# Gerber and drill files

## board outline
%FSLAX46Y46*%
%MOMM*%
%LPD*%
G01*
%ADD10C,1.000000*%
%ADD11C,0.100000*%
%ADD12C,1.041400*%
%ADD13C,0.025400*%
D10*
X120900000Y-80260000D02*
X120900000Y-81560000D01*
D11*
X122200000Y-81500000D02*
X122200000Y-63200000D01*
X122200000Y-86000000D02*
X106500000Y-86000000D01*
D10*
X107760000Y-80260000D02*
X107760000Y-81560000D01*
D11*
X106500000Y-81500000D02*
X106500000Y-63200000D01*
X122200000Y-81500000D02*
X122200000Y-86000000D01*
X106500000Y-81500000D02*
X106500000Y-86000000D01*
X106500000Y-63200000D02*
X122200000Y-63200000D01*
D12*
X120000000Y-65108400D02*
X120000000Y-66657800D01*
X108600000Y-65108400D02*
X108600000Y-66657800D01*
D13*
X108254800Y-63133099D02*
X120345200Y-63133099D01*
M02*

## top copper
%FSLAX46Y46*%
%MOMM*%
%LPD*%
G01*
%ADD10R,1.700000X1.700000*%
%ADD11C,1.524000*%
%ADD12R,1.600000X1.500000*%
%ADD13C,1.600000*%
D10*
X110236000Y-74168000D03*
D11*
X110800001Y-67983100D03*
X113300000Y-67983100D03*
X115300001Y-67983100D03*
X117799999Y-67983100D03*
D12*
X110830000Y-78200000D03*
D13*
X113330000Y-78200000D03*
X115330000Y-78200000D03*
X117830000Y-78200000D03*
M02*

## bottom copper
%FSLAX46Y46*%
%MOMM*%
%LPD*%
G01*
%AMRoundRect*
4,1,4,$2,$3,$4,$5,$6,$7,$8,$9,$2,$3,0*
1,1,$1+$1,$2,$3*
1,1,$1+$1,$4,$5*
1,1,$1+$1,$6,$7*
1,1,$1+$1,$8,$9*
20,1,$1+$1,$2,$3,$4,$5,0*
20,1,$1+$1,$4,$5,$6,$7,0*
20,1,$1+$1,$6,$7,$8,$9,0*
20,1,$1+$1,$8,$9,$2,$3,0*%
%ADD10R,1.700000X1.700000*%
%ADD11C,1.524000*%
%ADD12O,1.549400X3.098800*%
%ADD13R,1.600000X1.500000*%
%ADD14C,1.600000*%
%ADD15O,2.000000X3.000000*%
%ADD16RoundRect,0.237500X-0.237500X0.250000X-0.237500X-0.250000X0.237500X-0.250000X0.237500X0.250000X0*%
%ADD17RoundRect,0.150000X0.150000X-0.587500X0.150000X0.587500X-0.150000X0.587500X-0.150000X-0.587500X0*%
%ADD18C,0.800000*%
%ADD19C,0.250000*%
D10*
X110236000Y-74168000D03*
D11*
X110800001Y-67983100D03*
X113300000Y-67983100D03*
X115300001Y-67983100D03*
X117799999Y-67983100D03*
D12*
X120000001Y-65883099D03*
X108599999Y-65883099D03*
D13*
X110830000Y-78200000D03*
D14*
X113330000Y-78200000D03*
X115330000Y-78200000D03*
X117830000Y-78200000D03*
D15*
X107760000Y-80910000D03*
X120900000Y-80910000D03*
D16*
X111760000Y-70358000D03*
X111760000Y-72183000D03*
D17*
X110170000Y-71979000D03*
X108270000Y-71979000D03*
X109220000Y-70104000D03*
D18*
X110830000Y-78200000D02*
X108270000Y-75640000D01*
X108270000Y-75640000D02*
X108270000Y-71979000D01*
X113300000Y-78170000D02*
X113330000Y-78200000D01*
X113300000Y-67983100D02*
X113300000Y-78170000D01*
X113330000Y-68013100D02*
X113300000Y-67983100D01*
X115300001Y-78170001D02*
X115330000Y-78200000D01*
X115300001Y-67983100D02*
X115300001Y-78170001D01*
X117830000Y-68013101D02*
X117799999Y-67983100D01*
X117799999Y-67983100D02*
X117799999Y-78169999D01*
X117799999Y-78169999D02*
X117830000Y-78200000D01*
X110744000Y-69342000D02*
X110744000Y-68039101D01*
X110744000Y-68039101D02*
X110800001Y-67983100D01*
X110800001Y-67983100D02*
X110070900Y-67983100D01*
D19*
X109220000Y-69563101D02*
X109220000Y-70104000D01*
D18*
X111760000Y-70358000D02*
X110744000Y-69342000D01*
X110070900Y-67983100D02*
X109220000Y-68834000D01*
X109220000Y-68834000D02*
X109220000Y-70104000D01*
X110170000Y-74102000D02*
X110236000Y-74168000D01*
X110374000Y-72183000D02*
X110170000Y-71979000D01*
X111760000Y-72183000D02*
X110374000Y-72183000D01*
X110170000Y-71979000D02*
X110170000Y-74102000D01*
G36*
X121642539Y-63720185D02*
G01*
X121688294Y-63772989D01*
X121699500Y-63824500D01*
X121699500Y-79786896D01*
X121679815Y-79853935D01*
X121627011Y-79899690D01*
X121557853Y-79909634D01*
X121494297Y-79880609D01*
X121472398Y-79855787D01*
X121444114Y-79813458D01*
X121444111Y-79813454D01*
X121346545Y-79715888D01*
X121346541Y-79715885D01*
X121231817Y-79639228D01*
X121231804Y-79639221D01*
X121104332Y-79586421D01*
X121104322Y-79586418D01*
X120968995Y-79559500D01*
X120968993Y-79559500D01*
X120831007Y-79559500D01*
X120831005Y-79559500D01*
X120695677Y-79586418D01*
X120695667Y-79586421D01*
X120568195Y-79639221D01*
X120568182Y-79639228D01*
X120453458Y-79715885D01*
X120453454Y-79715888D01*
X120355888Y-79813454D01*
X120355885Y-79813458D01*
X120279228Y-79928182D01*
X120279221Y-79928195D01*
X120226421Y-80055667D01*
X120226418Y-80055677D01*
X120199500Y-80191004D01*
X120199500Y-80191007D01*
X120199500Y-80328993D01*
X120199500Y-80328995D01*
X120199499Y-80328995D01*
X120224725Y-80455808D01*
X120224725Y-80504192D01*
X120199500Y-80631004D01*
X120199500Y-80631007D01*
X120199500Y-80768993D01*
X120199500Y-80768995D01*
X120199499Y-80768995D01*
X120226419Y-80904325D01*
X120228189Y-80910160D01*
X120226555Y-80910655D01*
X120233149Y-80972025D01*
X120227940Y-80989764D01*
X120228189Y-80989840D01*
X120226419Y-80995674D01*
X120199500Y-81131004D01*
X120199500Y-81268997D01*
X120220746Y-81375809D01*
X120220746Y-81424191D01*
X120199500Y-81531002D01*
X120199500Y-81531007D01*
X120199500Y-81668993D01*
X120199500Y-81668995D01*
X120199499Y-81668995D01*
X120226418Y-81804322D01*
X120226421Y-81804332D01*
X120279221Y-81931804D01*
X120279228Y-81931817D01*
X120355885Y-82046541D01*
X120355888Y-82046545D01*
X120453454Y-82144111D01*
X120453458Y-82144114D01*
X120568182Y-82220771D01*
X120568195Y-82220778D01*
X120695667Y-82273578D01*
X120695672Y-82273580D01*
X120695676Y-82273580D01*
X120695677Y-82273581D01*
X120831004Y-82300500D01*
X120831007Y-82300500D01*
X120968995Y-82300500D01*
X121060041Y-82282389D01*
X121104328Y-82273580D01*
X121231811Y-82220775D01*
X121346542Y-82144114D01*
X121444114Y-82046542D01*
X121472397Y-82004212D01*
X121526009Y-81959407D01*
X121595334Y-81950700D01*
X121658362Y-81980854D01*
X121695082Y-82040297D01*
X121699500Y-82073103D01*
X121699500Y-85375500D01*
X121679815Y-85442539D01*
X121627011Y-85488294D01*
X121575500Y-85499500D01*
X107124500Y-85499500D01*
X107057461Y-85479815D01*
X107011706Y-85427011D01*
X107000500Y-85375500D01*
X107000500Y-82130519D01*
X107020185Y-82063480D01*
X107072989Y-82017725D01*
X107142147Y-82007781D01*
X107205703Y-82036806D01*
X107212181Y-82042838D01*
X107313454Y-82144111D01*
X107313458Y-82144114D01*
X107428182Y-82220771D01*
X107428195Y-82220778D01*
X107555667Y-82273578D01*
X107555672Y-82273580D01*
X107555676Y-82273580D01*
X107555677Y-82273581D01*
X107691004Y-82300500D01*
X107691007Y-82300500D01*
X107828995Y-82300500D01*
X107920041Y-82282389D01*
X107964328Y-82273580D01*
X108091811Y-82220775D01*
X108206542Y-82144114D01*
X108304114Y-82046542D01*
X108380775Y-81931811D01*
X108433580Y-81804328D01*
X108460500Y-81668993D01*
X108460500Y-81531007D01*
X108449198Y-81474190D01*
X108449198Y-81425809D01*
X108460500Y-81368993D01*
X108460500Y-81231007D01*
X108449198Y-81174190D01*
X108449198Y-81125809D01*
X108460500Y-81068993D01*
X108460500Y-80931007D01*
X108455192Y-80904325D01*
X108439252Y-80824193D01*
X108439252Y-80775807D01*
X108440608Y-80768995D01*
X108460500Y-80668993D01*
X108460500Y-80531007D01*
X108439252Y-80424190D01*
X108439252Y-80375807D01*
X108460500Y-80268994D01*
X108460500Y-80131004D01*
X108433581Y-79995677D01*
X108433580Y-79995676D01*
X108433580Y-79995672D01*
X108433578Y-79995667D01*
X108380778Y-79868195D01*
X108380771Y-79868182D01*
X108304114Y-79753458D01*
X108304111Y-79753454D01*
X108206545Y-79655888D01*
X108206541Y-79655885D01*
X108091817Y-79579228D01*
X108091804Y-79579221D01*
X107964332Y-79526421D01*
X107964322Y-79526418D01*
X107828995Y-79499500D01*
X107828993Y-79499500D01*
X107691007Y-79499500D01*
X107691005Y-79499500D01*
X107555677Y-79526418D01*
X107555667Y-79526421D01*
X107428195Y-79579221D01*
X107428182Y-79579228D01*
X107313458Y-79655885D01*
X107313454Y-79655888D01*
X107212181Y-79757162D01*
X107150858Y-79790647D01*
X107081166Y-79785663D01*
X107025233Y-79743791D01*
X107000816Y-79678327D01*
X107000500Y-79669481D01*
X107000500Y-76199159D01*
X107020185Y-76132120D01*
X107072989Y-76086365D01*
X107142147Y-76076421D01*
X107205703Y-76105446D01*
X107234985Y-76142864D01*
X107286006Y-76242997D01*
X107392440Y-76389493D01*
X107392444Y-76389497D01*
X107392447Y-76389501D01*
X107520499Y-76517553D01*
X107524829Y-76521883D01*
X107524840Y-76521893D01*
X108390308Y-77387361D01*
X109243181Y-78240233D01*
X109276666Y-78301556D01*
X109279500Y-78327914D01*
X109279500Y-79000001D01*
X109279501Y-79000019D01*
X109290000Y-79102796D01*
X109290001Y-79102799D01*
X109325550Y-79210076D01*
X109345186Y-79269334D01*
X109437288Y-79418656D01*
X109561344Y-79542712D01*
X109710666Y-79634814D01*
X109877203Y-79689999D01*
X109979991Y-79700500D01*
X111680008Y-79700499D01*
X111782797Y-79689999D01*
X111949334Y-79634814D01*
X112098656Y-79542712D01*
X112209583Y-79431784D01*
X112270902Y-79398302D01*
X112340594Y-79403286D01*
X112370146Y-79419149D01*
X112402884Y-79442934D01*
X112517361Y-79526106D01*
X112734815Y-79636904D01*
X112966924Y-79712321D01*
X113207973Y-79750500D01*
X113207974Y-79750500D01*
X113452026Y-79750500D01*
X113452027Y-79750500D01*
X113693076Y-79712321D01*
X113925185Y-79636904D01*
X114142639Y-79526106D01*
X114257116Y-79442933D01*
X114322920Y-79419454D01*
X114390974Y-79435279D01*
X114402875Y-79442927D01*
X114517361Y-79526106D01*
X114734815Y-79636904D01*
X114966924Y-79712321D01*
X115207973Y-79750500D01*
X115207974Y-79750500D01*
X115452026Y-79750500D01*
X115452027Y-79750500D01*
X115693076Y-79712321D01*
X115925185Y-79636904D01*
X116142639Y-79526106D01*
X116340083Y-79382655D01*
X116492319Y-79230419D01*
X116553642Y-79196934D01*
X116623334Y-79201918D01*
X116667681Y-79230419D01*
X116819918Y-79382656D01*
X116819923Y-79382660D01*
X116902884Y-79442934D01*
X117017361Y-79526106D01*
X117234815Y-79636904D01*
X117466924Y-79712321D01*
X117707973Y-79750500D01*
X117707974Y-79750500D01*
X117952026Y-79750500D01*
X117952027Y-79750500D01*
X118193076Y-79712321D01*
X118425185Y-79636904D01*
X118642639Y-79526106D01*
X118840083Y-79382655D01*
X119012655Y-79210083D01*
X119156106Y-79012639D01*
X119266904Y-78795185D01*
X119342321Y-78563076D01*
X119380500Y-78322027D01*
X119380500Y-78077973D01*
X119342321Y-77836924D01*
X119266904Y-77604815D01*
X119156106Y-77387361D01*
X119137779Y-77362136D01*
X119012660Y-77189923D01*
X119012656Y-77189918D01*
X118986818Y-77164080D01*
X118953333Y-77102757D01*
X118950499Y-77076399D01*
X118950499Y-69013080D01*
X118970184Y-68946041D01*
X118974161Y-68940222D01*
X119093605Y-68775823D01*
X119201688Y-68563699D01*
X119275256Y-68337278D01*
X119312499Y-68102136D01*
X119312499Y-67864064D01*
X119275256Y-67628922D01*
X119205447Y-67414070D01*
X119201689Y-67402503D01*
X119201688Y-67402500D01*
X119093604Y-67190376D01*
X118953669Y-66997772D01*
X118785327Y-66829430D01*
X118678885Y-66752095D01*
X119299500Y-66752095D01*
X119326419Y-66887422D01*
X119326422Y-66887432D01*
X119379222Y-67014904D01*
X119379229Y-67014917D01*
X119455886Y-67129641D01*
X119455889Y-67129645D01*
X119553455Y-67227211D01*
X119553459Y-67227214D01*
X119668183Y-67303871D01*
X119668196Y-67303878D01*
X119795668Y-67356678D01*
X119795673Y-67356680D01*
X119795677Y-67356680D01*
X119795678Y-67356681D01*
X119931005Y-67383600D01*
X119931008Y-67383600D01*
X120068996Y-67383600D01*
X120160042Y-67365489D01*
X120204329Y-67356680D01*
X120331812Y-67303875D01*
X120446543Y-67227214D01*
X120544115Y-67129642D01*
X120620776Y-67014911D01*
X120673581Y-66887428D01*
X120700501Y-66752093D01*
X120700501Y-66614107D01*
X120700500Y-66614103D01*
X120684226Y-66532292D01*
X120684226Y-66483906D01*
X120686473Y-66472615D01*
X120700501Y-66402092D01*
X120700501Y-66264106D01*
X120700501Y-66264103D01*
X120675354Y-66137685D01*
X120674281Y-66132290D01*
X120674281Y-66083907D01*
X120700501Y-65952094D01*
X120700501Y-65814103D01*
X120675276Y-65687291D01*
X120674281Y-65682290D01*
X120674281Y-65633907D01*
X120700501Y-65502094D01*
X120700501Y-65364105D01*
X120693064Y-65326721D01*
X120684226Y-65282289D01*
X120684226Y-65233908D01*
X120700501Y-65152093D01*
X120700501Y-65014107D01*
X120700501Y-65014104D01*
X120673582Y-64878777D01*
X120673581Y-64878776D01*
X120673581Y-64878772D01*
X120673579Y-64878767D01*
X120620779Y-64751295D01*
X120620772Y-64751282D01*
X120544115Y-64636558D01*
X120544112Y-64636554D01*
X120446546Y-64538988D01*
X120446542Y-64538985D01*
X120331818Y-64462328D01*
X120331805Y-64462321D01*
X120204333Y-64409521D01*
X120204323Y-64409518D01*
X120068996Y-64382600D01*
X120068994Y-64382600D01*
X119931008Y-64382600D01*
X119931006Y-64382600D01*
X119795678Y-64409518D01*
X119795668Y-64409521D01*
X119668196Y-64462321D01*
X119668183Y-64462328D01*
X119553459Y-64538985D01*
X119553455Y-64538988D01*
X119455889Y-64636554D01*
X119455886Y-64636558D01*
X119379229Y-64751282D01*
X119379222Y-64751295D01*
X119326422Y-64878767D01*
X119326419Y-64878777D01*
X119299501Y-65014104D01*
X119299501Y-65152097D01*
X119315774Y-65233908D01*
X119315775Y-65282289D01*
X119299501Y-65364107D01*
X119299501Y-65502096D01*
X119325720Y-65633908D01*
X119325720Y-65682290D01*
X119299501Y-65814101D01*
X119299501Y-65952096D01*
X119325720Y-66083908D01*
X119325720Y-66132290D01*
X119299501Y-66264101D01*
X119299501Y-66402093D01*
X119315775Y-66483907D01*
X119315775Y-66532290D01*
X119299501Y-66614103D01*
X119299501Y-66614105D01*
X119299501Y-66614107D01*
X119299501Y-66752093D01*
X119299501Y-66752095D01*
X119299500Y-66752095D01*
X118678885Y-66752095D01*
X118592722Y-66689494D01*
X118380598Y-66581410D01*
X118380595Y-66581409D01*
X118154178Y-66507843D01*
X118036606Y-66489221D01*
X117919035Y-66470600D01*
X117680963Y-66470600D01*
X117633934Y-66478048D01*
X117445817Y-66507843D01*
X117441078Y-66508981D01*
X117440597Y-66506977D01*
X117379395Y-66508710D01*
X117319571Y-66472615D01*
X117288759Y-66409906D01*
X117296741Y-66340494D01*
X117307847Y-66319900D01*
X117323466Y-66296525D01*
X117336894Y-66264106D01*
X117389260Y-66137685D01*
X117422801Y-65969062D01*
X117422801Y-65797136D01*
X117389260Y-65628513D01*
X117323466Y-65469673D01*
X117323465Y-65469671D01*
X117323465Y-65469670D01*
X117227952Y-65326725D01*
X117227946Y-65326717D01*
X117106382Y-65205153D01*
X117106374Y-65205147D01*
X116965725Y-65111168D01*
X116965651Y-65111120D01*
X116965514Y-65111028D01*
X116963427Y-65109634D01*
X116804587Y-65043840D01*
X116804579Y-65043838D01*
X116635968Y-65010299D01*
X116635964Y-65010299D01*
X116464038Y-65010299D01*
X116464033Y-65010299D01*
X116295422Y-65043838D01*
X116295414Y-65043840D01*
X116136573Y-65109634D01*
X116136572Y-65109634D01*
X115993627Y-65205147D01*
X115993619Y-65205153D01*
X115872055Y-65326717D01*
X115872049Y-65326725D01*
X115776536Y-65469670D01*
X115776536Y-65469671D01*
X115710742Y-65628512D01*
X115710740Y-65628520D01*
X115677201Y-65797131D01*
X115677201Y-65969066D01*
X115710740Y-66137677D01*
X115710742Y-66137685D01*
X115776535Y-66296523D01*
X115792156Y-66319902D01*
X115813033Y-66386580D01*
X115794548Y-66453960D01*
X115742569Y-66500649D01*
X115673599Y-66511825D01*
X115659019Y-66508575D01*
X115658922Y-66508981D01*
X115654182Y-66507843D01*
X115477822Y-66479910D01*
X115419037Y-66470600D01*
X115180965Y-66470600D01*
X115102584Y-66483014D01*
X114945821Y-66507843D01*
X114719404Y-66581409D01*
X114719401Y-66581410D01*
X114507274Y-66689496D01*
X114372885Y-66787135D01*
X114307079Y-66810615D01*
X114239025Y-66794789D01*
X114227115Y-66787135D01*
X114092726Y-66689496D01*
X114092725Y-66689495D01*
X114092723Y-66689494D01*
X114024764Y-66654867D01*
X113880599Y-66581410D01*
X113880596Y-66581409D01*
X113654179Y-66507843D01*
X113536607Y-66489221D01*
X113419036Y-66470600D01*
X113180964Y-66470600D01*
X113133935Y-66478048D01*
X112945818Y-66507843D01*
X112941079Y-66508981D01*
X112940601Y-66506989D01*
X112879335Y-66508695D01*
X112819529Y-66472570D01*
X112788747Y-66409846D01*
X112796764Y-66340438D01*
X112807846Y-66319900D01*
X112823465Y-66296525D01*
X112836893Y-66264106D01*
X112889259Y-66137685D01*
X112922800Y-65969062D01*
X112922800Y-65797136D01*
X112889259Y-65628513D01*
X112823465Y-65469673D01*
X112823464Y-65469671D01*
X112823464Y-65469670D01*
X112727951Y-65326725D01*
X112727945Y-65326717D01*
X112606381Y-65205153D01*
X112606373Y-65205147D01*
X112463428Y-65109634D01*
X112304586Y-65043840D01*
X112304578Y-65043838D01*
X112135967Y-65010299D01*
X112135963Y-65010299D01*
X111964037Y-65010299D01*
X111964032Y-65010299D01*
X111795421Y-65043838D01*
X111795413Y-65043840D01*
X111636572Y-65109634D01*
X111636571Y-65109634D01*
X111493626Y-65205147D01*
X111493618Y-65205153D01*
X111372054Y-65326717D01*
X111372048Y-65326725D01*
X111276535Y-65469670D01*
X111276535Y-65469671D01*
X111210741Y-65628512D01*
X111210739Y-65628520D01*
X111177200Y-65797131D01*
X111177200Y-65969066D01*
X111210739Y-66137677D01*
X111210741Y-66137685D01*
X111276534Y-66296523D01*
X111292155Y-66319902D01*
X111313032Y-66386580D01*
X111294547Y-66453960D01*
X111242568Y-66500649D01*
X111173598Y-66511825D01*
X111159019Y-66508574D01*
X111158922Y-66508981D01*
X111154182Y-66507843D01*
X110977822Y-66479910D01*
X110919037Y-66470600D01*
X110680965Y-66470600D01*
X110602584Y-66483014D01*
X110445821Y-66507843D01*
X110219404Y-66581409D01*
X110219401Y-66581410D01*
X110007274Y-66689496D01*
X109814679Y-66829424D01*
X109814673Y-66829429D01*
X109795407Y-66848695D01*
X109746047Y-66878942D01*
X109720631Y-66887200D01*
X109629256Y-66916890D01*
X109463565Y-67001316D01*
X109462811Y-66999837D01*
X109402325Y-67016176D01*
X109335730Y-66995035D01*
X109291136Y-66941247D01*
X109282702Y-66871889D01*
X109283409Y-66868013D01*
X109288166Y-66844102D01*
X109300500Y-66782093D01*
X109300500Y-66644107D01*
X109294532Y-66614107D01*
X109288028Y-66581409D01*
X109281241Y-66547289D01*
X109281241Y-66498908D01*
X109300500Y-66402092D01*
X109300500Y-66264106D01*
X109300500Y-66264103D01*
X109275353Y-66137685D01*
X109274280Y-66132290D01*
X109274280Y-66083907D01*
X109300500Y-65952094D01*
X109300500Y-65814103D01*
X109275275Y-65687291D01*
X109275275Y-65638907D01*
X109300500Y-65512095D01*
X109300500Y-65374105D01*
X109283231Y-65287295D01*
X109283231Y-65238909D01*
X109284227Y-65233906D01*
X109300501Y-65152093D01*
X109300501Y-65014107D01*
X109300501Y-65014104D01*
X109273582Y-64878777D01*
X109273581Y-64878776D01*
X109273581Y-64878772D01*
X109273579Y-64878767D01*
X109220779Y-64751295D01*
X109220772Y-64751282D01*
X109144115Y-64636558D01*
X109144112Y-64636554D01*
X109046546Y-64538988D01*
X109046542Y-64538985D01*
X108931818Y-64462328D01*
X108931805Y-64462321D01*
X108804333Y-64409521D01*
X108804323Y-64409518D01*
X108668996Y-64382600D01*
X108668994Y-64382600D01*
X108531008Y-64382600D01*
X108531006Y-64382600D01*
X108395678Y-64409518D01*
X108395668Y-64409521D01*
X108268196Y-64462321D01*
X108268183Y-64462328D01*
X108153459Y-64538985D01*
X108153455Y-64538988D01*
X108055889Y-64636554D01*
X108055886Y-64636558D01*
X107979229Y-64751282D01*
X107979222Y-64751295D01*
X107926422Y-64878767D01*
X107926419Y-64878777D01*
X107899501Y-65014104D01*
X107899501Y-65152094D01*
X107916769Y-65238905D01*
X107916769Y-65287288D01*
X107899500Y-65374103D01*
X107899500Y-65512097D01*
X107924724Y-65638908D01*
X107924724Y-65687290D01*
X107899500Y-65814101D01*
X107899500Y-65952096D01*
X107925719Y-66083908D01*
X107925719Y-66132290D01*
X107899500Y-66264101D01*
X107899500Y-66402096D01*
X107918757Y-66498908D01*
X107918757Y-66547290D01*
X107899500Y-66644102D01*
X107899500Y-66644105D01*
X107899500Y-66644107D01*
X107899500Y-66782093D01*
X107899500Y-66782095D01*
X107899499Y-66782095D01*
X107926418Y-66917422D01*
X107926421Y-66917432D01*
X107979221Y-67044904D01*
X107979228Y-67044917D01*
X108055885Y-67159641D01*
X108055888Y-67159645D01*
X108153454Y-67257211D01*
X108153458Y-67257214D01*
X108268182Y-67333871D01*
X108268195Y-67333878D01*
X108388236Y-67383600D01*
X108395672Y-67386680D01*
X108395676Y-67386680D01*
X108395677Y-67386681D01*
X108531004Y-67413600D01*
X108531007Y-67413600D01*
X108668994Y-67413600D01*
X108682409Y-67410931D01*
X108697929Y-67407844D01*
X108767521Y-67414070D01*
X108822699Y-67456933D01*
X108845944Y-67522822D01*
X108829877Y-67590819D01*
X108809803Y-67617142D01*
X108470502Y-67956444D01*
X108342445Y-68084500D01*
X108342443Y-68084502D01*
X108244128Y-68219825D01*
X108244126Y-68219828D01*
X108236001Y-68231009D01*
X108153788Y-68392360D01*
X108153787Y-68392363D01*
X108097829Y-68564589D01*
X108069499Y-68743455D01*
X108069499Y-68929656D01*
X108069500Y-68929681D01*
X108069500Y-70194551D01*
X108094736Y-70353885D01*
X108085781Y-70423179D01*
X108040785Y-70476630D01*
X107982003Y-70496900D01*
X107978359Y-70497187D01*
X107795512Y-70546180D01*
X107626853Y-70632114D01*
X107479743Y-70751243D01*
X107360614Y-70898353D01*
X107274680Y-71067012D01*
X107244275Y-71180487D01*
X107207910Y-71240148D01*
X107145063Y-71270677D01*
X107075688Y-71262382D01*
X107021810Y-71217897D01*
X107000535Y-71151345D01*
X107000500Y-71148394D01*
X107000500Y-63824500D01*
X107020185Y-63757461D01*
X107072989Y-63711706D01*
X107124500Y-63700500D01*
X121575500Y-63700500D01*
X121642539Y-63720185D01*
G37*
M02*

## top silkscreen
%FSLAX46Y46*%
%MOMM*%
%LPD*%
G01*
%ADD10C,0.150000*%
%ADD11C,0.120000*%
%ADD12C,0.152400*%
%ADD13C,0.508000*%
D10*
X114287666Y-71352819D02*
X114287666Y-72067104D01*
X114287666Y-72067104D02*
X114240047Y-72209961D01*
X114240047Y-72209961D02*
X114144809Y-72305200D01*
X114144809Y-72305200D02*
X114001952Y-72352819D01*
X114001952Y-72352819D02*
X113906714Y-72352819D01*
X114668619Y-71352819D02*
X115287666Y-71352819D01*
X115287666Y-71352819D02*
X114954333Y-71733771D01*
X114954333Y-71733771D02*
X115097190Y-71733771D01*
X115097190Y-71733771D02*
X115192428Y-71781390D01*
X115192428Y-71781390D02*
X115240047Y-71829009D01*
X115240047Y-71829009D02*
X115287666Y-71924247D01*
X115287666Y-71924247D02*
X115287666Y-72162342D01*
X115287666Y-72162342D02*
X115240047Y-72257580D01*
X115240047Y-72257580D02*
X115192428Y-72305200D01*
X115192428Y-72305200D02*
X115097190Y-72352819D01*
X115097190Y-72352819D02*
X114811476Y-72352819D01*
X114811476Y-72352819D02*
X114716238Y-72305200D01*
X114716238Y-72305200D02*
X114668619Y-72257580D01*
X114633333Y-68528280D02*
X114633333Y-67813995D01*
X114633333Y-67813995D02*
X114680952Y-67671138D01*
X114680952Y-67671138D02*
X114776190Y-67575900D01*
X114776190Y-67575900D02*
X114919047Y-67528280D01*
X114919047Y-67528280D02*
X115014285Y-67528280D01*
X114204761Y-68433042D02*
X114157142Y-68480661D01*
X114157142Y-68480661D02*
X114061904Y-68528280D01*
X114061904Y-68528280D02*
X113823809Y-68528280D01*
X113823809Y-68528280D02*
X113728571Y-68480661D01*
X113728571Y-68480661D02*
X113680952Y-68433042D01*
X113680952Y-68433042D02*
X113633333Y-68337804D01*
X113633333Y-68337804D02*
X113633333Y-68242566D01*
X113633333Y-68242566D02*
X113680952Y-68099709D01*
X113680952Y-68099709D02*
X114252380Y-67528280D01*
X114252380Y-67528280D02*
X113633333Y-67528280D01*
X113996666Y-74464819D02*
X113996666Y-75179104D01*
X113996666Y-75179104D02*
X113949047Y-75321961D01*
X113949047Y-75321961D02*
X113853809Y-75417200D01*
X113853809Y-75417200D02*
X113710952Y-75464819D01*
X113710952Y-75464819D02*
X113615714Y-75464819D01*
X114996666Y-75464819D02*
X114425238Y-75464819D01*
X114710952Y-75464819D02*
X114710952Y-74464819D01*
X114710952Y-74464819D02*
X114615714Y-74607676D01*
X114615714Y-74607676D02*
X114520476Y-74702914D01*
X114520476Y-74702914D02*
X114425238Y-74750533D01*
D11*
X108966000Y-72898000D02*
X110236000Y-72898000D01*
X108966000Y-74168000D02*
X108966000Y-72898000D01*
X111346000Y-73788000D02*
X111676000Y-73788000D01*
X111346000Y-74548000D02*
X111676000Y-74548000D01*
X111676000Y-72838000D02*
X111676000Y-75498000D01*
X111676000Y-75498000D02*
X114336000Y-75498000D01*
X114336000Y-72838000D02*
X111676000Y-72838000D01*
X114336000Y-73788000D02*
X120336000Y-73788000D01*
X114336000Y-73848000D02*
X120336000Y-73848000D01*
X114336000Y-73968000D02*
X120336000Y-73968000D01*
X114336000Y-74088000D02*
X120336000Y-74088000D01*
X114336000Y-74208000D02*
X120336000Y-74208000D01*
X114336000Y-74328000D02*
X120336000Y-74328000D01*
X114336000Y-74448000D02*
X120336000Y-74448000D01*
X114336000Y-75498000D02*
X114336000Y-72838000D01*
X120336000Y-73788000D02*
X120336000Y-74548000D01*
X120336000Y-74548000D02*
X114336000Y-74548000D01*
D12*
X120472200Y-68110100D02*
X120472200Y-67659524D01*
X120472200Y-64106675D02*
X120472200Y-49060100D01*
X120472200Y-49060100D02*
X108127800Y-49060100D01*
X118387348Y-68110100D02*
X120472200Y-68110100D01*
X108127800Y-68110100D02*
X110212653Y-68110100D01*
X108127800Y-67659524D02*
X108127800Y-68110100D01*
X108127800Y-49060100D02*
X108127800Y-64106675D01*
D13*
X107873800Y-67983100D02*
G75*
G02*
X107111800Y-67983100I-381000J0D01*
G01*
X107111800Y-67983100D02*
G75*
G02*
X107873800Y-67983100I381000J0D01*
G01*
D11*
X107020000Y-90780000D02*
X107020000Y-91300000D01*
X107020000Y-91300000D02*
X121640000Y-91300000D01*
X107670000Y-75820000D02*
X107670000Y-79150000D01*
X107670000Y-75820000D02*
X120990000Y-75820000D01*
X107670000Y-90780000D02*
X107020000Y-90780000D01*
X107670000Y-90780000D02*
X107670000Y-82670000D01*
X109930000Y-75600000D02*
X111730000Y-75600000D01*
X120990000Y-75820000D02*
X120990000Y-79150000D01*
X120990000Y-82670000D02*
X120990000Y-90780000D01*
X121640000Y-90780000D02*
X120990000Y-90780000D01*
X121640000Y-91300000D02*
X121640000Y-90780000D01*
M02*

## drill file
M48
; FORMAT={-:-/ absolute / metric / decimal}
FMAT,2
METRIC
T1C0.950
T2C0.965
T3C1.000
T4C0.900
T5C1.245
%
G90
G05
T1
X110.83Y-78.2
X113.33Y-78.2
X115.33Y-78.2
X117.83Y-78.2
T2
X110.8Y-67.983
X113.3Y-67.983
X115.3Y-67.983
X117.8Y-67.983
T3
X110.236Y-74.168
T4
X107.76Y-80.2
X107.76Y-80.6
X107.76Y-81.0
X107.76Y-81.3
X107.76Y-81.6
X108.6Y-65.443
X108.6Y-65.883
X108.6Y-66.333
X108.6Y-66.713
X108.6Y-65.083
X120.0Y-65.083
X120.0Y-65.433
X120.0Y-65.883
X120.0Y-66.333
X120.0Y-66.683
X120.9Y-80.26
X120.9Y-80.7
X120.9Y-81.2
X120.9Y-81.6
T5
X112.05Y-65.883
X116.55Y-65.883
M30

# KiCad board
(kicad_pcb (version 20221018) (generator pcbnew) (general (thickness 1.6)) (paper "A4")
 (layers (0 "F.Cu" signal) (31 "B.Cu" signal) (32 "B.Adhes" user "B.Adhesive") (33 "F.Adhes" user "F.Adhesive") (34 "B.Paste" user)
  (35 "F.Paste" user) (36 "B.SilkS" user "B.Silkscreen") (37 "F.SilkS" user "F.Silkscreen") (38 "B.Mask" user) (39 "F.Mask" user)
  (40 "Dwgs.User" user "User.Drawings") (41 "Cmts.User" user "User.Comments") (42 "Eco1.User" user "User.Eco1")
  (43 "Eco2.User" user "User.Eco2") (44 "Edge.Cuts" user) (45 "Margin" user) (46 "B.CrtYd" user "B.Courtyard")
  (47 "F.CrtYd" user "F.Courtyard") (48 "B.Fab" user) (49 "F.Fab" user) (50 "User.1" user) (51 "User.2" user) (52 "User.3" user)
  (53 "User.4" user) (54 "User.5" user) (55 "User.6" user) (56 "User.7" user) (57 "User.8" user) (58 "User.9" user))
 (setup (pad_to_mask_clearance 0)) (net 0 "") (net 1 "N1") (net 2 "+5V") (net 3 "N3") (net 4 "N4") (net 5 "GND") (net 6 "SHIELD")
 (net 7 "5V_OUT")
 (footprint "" (layer "F.Cu") (at 120.9 78.74)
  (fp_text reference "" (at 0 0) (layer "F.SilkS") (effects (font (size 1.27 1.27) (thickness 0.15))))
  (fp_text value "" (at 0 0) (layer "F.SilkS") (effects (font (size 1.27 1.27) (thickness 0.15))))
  (pad "" np_thru_hole circle (at 0 1.96 180) (size 0.9 0.9) (drill 0.9) (layers "F&B.Cu" "*.Mask")))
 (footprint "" (layer "F.Cu") (at 120.9 79.24)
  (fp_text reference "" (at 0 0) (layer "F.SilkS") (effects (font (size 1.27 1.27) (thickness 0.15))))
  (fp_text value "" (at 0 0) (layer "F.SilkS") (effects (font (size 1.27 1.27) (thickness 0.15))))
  (pad "" np_thru_hole circle (at 0 1.96 180) (size 0.9 0.9) (drill 0.9) (layers "F&B.Cu" "*.Mask")))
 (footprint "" (layer "F.Cu") (at 104.2 78.24)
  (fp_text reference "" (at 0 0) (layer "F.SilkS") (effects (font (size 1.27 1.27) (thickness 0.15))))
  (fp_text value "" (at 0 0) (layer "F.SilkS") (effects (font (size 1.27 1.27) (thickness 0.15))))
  (pad "" np_thru_hole circle (at 3.56 1.96 180) (size 0.9 0.9) (drill 0.9) (layers "F&B.Cu" "*.Mask")))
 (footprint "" (layer "F.Cu") (at 120.9 79.64)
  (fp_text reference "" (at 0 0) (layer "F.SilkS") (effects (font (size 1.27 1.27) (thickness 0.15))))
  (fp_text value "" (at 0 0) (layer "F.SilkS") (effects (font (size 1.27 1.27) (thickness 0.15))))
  (pad "" np_thru_hole circle (at 0 1.96 180) (size 0.9 0.9) (drill 0.9) (layers "F&B.Cu" "*.Mask")))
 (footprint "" (layer "F.Cu") (at 104.2 78.64)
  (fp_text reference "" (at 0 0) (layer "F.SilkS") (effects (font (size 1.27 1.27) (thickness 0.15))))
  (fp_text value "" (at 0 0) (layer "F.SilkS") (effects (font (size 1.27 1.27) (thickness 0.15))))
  (pad "" np_thru_hole circle (at 3.56 1.96 180) (size 0.9 0.9) (drill 0.9) (layers "F&B.Cu" "*.Mask")))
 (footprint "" (layer "F.Cu") (at 120.9 78.3)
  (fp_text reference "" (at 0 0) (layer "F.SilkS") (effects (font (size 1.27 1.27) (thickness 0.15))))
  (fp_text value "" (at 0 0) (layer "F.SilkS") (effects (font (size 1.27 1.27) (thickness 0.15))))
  (pad "" np_thru_hole circle (at 0 1.96 180) (size 0.9 0.9) (drill 0.9) (layers "F&B.Cu" "*.Mask")))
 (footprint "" (layer "F.Cu") (at 104.2 79.34)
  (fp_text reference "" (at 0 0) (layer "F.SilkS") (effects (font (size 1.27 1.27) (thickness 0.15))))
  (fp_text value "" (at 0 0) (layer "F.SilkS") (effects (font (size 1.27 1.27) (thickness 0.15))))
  (pad "" np_thru_hole circle (at 3.56 1.96 180) (size 0.9 0.9) (drill 0.9) (layers "F&B.Cu" "*.Mask")))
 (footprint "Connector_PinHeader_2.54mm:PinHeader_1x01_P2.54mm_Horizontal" (layer "F.Cu") (at 110.236 74.168)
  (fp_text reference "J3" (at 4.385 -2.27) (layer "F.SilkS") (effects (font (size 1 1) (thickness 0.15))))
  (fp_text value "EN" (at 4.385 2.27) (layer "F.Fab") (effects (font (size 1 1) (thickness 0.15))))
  (fp_line (start -1.27 -1.27) (end 0 -1.27) (stroke (width 0.12) (type solid)) (layer "F.SilkS"))
  (fp_line (start -1.27 0) (end -1.27 -1.27) (stroke (width 0.12) (type solid)) (layer "F.SilkS"))
  (fp_line (start 1.11 -0.38) (end 1.44 -0.38) (stroke (width 0.12) (type solid)) (layer "F.SilkS"))
  (fp_line (start 1.11 0.38) (end 1.44 0.38) (stroke (width 0.12) (type solid)) (layer "F.SilkS"))
  (fp_line (start 1.44 -1.33) (end 1.44 1.33) (stroke (width 0.12) (type solid)) (layer "F.SilkS"))
  (fp_line (start 1.44 1.33) (end 4.1 1.33) (stroke (width 0.12) (type solid)) (layer "F.SilkS"))
  (fp_line (start 4.1 -1.33) (end 1.44 -1.33) (stroke (width 0.12) (type solid)) (layer "F.SilkS"))
  (fp_line (start 4.1 -0.38) (end 10.1 -0.38) (stroke (width 0.12) (type solid)) (layer "F.SilkS"))
  (fp_line (start 4.1 -0.32) (end 10.1 -0.32) (stroke (width 0.12) (type solid)) (layer "F.SilkS"))
  (fp_line (start 4.1 -0.2) (end 10.1 -0.2) (stroke (width 0.12) (type solid)) (layer "F.SilkS"))
  (fp_line (start 4.1 -0.08) (end 10.1 -0.08) (stroke (width 0.12) (type solid)) (layer "F.SilkS"))
  (fp_line (start 4.1 0.04) (end 10.1 0.04) (stroke (width 0.12) (type solid)) (layer "F.SilkS"))
  (fp_line (start 4.1 0.16) (end 10.1 0.16) (stroke (width 0.12) (type solid)) (layer "F.SilkS"))
  (fp_line (start 4.1 0.28) (end 10.1 0.28) (stroke (width 0.12) (type solid)) (layer "F.SilkS"))
  (fp_line (start 4.1 1.33) (end 4.1 -1.33) (stroke (width 0.12) (type solid)) (layer "F.SilkS"))
  (fp_line (start 10.1 -0.38) (end 10.1 0.38) (stroke (width 0.12) (type solid)) (layer "F.SilkS"))
  (fp_line (start 10.1 0.38) (end 4.1 0.38) (stroke (width 0.12) (type solid)) (layer "F.SilkS"))
  (pad "1" thru_hole rect (at 0 0) (size 1.7 1.7) (drill 1) (layers "*.Cu" "*.Mask") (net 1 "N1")))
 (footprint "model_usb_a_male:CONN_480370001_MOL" (layer "F.Cu") (at 110.800001 67.9831 180)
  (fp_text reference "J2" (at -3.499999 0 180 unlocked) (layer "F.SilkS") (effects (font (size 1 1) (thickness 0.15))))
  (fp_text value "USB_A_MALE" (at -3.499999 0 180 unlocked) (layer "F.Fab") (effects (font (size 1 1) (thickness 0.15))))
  (fp_line (start -9.672199 -0.127) (end -9.672199 0.323576) (stroke (width 0.1524) (type solid)) (layer "F.SilkS"))
  (fp_line (start -9.672199 3.876425) (end -9.672199 18.923) (stroke (width 0.1524) (type solid)) (layer "F.SilkS"))
  (fp_line (start -9.672199 18.923) (end 2.672201 18.923) (stroke (width 0.1524) (type solid)) (layer "F.SilkS"))
  (fp_line (start -7.587347 -0.127) (end -9.672199 -0.127) (stroke (width 0.1524) (type solid)) (layer "F.SilkS"))
  (fp_line (start 2.672201 -0.127) (end 0.587348 -0.127) (stroke (width 0.1524) (type solid)) (layer "F.SilkS"))
  (fp_line (start 2.672201 0.323576) (end 2.672201 -0.127) (stroke (width 0.1524) (type solid)) (layer "F.SilkS"))
  (fp_line (start 2.672201 18.923) (end 2.672201 3.876425) (stroke (width 0.1524) (type solid)) (layer "F.SilkS"))
  (fp_circle (center 3.307201 0) (end 3.688201 0) (stroke (width 0.508) (type solid)) (fill none) (layer "F.SilkS"))
  (fp_line (start -9.199999 2.8747) (end -9.199999 1.3253) (stroke (width 1.0414) (type solid)) (layer "Edge.Cuts"))
  (fp_line (start 2.200001 2.8747) (end 2.200001 1.3253) (stroke (width 1.0414) (type solid)) (layer "Edge.Cuts"))
  (fp_line (start 2.545201 4.850001) (end -9.545199 4.850001) (stroke (width 0.0254) (type solid)) (layer "Edge.Cuts"))
  (pad "" np_thru_hole circle (at -9.2 1.3 180) (size 0.9 0.9) (drill 0.9) (layers "F&B.Cu" "*.Mask"))
  (pad "" np_thru_hole circle (at -9.2 1.650001 180) (size 0.9 0.9) (drill 0.9) (layers "F&B.Cu" "*.Mask"))
  (pad "" np_thru_hole circle (at -9.2 2.100001 180) (size 0.9 0.9) (drill 0.9) (layers "F&B.Cu" "*.Mask"))
  (pad "" np_thru_hole circle (at -9.2 2.550001 180) (size 0.9 0.9) (drill 0.9) (layers "F&B.Cu" "*.Mask"))
  (pad "" np_thru_hole circle (at -9.2 2.9 180) (size 0.9 0.9) (drill 0.9) (layers "F&B.Cu" "*.Mask"))
  (pad "" np_thru_hole circle (at -5.75 2.100001 180) (size 1.2446 1.2446) (drill 1.2446) (layers))
  (pad "" np_thru_hole circle (at -1.249999 2.100001 180) (size 1.2446 1.2446) (drill 1.2446) (layers))
  (pad "" np_thru_hole circle (at 2.2 2.9 180) (size 0.9 0.9) (drill 0.9) (layers "F&B.Cu" "*.Mask"))
  (pad "" np_thru_hole circle (at 2.200001 1.27 180) (size 0.9 0.9) (drill 0.9) (layers "F&B.Cu" "*.Mask"))
  (pad "" np_thru_hole circle (at 2.200001 1.650001 180) (size 0.9 0.9) (drill 0.9) (layers "F&B.Cu" "*.Mask"))
  (pad "" np_thru_hole circle (at 2.200001 2.100001 180) (size 0.9 0.9) (drill 0.9) (layers "F&B.Cu" "*.Mask"))
  (pad "" np_thru_hole circle (at 2.200001 2.54 180) (size 0.9 0.9) (drill 0.9) (layers "F&B.Cu" "*.Mask"))
  (pad "1" thru_hole circle (at 0 0 180) (size 1.524 1.524) (drill 0.9652) (layers "*.Cu" "*.Mask") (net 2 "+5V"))
  (pad "2" thru_hole circle (at -2.499999 0 180) (size 1.524 1.524) (drill 0.9652) (layers "*.Cu" "*.Mask") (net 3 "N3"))
  (pad "3" thru_hole circle (at -4.5 0 180) (size 1.524 1.524) (drill 0.9652) (layers "*.Cu" "*.Mask") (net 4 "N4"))
  (pad "4" thru_hole circle (at -6.999998 0 180) (size 1.524 1.524) (drill 0.9652) (layers "*.Cu" "*.Mask") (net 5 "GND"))
  (pad "5" smd oval (at -9.2 2.100001 180) (size 1.5494 3.0988) (layers "B.Cu" "F.Paste" "F.Mask") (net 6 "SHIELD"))
  (pad "5" smd oval (at 2.200002 2.100001 180) (size 1.5494 3.0988) (layers "B.Cu" "F.Paste" "F.Mask") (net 6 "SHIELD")))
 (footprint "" (layer "F.Cu") (at 104.2 79.04)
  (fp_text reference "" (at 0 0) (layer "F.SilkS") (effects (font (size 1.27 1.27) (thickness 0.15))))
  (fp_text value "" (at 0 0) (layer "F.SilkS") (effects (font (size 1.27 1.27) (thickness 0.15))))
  (pad "" np_thru_hole circle (at 3.56 1.96 180) (size 0.9 0.9) (drill 0.9) (layers "F&B.Cu" "*.Mask")))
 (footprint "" (layer "F.Cu") (at 104.2 79.64)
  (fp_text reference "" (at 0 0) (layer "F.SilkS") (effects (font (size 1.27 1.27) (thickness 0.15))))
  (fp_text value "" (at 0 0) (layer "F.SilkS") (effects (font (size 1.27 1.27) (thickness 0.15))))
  (pad "" np_thru_hole circle (at 3.56 1.96 180) (size 0.9 0.9) (drill 0.9) (layers "F&B.Cu" "*.Mask")))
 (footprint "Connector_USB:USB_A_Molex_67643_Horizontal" (layer "F.Cu") (at 110.83 78.2)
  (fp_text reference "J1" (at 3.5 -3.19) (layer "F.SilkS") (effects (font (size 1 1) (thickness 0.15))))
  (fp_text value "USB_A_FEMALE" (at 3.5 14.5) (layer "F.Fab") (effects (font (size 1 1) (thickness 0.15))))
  (fp_line (start -3.81 12.58) (end -3.81 13.1) (stroke (width 0.12) (type solid)) (layer "F.SilkS"))
  (fp_line (start -3.81 13.1) (end 10.81 13.1) (stroke (width 0.12) (type solid)) (layer "F.SilkS"))
  (fp_line (start -3.16 -2.38) (end -3.16 0.95) (stroke (width 0.12) (type solid)) (layer "F.SilkS"))
  (fp_line (start -3.16 -2.38) (end 10.16 -2.38) (stroke (width 0.12) (type solid)) (layer "F.SilkS"))
  (fp_line (start -3.16 12.58) (end -3.81 12.58) (stroke (width 0.12) (type solid)) (layer "F.SilkS"))
  (fp_line (start -3.16 12.58) (end -3.16 4.47) (stroke (width 0.12) (type solid)) (layer "F.SilkS"))
  (fp_line (start -0.9 -2.6) (end 0.9 -2.6) (stroke (width 0.12) (type solid)) (layer "F.SilkS"))
  (fp_line (start 10.16 -2.38) (end 10.16 0.95) (stroke (width 0.12) (type solid)) (layer "F.SilkS"))
  (fp_line (start 10.16 4.47) (end 10.16 12.58) (stroke (width 0.12) (type solid)) (layer "F.SilkS"))
  (fp_line (start 10.81 12.58) (end 10.16 12.58) (stroke (width 0.12) (type solid)) (layer "F.SilkS"))
  (fp_line (start 10.81 13.1) (end 10.81 12.58) (stroke (width 0.12) (type solid)) (layer "F.SilkS"))
  (pad "1" thru_hole rect (at 0 0) (size 1.6 1.5) (drill 0.95) (layers "*.Cu" "*.Mask") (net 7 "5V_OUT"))
  (pad "2" thru_hole circle (at 2.5 0) (size 1.6 1.6) (drill 0.95) (layers "*.Cu" "*.Mask") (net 3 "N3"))
  (pad "3" thru_hole circle (at 4.5 0) (size 1.6 1.6) (drill 0.95) (layers "*.Cu" "*.Mask") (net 4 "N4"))
  (pad "4" thru_hole circle (at 7 0) (size 1.6 1.6) (drill 0.95) (layers "*.Cu" "*.Mask") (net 5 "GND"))
  (pad "5" smd oval (at -3.07 2.71) (size 2 3) (layers "B.Cu" "F.Paste" "F.Mask") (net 6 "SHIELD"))
  (pad "5" smd oval (at 10.07 2.71) (size 2 3) (layers "B.Cu" "F.Paste" "F.Mask") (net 6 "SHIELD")))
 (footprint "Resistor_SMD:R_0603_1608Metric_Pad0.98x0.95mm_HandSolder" (layer "B.Cu") (at 111.76 71.2705 -90)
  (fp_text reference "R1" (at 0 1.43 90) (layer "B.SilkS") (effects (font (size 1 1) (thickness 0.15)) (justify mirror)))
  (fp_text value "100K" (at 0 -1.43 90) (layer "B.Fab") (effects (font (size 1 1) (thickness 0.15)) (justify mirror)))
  (pad "1" smd roundrect (at -0.9125 0 270) (size 0.975 0.95) (layers "B.Cu" "B.Paste" "B.Mask") (roundrect_rratio 0.25) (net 2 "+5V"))
  (pad "2" smd roundrect (at 0.9125 0 270) (size 0.975 0.95) (layers "B.Cu" "B.Paste" "B.Mask") (roundrect_rratio 0.25) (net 1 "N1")))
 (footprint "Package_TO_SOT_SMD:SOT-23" (layer "B.Cu") (at 109.22 71.0415 90)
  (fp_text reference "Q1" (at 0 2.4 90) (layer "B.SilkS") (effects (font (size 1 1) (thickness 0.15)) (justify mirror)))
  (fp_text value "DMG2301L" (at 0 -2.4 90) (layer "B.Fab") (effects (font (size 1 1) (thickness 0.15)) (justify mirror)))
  (pad "1" smd roundrect (at -0.9375 0.95 90) (size 1.475 0.6) (layers "B.Cu" "B.Paste" "B.Mask") (roundrect_rratio 0.25) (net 1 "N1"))
  (pad "2" smd roundrect (at -0.9375 -0.95 90) (size 1.475 0.6) (layers "B.Cu" "B.Paste" "B.Mask") (roundrect_rratio 0.25) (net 7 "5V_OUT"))
  (pad "3" smd roundrect (at 0.9375 0 90) (size 1.475 0.6) (layers "B.Cu" "B.Paste" "B.Mask") (roundrect_rratio 0.25) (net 2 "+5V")))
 (gr_line (start 120.9 80.26) (end 120.9 81.56) (stroke (width 1) (type default)) (layer "Edge.Cuts"))
 (gr_line (start 122.2 81.5) (end 122.2 63.2) (stroke (width 0.1) (type default)) (layer "Edge.Cuts"))
 (gr_line (start 122.2 86) (end 106.5 86) (stroke (width 0.1) (type default)) (layer "Edge.Cuts"))
 (gr_line (start 107.76 80.26) (end 107.76 81.56) (stroke (width 1) (type default)) (layer "Edge.Cuts"))
 (gr_line (start 106.5 81.5) (end 106.5 63.2) (stroke (width 0.1) (type default)) (layer "Edge.Cuts"))
 (gr_line (start 122.2 81.5) (end 122.2 86) (stroke (width 0.1) (type default)) (layer "Edge.Cuts"))
 (gr_line (start 106.5 81.5) (end 106.5 86) (stroke (width 0.1) (type default)) (layer "Edge.Cuts"))
 (gr_line (start 106.5 63.2) (end 122.2 63.2) (stroke (width 0.1) (type default)) (layer "Edge.Cuts"))
 (segment (start 110.83 78.2) (end 108.27 75.64) (width 0.8) (layer "B.Cu") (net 7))
 (segment (start 108.27 75.64) (end 108.27 71.979) (width 0.8) (layer "B.Cu") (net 7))
 (segment (start 113.3 78.17) (end 113.33 78.2) (width 0.8) (layer "B.Cu") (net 3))
 (segment (start 113.3 67.9831) (end 113.3 78.17) (width 0.8) (layer "B.Cu") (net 3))
 (segment (start 113.33 68.0131) (end 113.3 67.9831) (width 0.8) (layer "B.Cu") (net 3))
 (segment (start 115.300001 78.170001) (end 115.33 78.2) (width 0.8) (layer "B.Cu") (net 4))
 (segment (start 115.300001 67.9831) (end 115.300001 78.170001) (width 0.8) (layer "B.Cu") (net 4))
 (segment (start 117.83 68.013101) (end 117.799999 67.9831) (width 0.8) (layer "B.Cu") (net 5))
 (segment (start 117.799999 67.9831) (end 117.799999 78.169999) (width 0.8) (layer "B.Cu") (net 5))
 (segment (start 117.799999 78.169999) (end 117.83 78.2) (width 0.8) (layer "B.Cu") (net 5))
 (segment (start 110.744 69.342) (end 110.744 68.039101) (width 0.8) (layer "B.Cu") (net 2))
 (segment (start 110.744 68.039101) (end 110.800001 67.9831) (width 0.8) (layer "B.Cu") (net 2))
 (segment (start 110.800001 67.9831) (end 110.0709 67.9831) (width 0.8) (layer "B.Cu") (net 2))
 (segment (start 109.22 69.563101) (end 109.22 70.104) (width 0.25) (layer "B.Cu") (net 2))
 (segment (start 111.76 70.358) (end 110.744 69.342) (width 0.8) (layer "B.Cu") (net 2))
 (segment (start 110.0709 67.9831) (end 109.22 68.834) (width 0.8) (layer "B.Cu") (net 2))
 (segment (start 109.22 68.834) (end 109.22 70.104) (width 0.8) (layer "B.Cu") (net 2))
 (segment (start 110.17 74.102) (end 110.236 74.168) (width 0.8) (layer "B.Cu") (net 1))
 (segment (start 110.374 72.183) (end 110.17 71.979) (width 0.8) (layer "B.Cu") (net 1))
 (segment (start 111.76 72.183) (end 110.374 72.183) (width 0.8) (layer "B.Cu") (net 1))
 (segment (start 110.17 71.979) (end 110.17 74.102) (width 0.8) (layer "B.Cu") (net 1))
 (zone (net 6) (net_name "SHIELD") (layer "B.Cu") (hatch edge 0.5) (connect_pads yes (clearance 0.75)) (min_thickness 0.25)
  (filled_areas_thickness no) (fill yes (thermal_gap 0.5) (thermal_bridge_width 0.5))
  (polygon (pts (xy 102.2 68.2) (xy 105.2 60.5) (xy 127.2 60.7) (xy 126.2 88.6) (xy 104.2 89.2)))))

